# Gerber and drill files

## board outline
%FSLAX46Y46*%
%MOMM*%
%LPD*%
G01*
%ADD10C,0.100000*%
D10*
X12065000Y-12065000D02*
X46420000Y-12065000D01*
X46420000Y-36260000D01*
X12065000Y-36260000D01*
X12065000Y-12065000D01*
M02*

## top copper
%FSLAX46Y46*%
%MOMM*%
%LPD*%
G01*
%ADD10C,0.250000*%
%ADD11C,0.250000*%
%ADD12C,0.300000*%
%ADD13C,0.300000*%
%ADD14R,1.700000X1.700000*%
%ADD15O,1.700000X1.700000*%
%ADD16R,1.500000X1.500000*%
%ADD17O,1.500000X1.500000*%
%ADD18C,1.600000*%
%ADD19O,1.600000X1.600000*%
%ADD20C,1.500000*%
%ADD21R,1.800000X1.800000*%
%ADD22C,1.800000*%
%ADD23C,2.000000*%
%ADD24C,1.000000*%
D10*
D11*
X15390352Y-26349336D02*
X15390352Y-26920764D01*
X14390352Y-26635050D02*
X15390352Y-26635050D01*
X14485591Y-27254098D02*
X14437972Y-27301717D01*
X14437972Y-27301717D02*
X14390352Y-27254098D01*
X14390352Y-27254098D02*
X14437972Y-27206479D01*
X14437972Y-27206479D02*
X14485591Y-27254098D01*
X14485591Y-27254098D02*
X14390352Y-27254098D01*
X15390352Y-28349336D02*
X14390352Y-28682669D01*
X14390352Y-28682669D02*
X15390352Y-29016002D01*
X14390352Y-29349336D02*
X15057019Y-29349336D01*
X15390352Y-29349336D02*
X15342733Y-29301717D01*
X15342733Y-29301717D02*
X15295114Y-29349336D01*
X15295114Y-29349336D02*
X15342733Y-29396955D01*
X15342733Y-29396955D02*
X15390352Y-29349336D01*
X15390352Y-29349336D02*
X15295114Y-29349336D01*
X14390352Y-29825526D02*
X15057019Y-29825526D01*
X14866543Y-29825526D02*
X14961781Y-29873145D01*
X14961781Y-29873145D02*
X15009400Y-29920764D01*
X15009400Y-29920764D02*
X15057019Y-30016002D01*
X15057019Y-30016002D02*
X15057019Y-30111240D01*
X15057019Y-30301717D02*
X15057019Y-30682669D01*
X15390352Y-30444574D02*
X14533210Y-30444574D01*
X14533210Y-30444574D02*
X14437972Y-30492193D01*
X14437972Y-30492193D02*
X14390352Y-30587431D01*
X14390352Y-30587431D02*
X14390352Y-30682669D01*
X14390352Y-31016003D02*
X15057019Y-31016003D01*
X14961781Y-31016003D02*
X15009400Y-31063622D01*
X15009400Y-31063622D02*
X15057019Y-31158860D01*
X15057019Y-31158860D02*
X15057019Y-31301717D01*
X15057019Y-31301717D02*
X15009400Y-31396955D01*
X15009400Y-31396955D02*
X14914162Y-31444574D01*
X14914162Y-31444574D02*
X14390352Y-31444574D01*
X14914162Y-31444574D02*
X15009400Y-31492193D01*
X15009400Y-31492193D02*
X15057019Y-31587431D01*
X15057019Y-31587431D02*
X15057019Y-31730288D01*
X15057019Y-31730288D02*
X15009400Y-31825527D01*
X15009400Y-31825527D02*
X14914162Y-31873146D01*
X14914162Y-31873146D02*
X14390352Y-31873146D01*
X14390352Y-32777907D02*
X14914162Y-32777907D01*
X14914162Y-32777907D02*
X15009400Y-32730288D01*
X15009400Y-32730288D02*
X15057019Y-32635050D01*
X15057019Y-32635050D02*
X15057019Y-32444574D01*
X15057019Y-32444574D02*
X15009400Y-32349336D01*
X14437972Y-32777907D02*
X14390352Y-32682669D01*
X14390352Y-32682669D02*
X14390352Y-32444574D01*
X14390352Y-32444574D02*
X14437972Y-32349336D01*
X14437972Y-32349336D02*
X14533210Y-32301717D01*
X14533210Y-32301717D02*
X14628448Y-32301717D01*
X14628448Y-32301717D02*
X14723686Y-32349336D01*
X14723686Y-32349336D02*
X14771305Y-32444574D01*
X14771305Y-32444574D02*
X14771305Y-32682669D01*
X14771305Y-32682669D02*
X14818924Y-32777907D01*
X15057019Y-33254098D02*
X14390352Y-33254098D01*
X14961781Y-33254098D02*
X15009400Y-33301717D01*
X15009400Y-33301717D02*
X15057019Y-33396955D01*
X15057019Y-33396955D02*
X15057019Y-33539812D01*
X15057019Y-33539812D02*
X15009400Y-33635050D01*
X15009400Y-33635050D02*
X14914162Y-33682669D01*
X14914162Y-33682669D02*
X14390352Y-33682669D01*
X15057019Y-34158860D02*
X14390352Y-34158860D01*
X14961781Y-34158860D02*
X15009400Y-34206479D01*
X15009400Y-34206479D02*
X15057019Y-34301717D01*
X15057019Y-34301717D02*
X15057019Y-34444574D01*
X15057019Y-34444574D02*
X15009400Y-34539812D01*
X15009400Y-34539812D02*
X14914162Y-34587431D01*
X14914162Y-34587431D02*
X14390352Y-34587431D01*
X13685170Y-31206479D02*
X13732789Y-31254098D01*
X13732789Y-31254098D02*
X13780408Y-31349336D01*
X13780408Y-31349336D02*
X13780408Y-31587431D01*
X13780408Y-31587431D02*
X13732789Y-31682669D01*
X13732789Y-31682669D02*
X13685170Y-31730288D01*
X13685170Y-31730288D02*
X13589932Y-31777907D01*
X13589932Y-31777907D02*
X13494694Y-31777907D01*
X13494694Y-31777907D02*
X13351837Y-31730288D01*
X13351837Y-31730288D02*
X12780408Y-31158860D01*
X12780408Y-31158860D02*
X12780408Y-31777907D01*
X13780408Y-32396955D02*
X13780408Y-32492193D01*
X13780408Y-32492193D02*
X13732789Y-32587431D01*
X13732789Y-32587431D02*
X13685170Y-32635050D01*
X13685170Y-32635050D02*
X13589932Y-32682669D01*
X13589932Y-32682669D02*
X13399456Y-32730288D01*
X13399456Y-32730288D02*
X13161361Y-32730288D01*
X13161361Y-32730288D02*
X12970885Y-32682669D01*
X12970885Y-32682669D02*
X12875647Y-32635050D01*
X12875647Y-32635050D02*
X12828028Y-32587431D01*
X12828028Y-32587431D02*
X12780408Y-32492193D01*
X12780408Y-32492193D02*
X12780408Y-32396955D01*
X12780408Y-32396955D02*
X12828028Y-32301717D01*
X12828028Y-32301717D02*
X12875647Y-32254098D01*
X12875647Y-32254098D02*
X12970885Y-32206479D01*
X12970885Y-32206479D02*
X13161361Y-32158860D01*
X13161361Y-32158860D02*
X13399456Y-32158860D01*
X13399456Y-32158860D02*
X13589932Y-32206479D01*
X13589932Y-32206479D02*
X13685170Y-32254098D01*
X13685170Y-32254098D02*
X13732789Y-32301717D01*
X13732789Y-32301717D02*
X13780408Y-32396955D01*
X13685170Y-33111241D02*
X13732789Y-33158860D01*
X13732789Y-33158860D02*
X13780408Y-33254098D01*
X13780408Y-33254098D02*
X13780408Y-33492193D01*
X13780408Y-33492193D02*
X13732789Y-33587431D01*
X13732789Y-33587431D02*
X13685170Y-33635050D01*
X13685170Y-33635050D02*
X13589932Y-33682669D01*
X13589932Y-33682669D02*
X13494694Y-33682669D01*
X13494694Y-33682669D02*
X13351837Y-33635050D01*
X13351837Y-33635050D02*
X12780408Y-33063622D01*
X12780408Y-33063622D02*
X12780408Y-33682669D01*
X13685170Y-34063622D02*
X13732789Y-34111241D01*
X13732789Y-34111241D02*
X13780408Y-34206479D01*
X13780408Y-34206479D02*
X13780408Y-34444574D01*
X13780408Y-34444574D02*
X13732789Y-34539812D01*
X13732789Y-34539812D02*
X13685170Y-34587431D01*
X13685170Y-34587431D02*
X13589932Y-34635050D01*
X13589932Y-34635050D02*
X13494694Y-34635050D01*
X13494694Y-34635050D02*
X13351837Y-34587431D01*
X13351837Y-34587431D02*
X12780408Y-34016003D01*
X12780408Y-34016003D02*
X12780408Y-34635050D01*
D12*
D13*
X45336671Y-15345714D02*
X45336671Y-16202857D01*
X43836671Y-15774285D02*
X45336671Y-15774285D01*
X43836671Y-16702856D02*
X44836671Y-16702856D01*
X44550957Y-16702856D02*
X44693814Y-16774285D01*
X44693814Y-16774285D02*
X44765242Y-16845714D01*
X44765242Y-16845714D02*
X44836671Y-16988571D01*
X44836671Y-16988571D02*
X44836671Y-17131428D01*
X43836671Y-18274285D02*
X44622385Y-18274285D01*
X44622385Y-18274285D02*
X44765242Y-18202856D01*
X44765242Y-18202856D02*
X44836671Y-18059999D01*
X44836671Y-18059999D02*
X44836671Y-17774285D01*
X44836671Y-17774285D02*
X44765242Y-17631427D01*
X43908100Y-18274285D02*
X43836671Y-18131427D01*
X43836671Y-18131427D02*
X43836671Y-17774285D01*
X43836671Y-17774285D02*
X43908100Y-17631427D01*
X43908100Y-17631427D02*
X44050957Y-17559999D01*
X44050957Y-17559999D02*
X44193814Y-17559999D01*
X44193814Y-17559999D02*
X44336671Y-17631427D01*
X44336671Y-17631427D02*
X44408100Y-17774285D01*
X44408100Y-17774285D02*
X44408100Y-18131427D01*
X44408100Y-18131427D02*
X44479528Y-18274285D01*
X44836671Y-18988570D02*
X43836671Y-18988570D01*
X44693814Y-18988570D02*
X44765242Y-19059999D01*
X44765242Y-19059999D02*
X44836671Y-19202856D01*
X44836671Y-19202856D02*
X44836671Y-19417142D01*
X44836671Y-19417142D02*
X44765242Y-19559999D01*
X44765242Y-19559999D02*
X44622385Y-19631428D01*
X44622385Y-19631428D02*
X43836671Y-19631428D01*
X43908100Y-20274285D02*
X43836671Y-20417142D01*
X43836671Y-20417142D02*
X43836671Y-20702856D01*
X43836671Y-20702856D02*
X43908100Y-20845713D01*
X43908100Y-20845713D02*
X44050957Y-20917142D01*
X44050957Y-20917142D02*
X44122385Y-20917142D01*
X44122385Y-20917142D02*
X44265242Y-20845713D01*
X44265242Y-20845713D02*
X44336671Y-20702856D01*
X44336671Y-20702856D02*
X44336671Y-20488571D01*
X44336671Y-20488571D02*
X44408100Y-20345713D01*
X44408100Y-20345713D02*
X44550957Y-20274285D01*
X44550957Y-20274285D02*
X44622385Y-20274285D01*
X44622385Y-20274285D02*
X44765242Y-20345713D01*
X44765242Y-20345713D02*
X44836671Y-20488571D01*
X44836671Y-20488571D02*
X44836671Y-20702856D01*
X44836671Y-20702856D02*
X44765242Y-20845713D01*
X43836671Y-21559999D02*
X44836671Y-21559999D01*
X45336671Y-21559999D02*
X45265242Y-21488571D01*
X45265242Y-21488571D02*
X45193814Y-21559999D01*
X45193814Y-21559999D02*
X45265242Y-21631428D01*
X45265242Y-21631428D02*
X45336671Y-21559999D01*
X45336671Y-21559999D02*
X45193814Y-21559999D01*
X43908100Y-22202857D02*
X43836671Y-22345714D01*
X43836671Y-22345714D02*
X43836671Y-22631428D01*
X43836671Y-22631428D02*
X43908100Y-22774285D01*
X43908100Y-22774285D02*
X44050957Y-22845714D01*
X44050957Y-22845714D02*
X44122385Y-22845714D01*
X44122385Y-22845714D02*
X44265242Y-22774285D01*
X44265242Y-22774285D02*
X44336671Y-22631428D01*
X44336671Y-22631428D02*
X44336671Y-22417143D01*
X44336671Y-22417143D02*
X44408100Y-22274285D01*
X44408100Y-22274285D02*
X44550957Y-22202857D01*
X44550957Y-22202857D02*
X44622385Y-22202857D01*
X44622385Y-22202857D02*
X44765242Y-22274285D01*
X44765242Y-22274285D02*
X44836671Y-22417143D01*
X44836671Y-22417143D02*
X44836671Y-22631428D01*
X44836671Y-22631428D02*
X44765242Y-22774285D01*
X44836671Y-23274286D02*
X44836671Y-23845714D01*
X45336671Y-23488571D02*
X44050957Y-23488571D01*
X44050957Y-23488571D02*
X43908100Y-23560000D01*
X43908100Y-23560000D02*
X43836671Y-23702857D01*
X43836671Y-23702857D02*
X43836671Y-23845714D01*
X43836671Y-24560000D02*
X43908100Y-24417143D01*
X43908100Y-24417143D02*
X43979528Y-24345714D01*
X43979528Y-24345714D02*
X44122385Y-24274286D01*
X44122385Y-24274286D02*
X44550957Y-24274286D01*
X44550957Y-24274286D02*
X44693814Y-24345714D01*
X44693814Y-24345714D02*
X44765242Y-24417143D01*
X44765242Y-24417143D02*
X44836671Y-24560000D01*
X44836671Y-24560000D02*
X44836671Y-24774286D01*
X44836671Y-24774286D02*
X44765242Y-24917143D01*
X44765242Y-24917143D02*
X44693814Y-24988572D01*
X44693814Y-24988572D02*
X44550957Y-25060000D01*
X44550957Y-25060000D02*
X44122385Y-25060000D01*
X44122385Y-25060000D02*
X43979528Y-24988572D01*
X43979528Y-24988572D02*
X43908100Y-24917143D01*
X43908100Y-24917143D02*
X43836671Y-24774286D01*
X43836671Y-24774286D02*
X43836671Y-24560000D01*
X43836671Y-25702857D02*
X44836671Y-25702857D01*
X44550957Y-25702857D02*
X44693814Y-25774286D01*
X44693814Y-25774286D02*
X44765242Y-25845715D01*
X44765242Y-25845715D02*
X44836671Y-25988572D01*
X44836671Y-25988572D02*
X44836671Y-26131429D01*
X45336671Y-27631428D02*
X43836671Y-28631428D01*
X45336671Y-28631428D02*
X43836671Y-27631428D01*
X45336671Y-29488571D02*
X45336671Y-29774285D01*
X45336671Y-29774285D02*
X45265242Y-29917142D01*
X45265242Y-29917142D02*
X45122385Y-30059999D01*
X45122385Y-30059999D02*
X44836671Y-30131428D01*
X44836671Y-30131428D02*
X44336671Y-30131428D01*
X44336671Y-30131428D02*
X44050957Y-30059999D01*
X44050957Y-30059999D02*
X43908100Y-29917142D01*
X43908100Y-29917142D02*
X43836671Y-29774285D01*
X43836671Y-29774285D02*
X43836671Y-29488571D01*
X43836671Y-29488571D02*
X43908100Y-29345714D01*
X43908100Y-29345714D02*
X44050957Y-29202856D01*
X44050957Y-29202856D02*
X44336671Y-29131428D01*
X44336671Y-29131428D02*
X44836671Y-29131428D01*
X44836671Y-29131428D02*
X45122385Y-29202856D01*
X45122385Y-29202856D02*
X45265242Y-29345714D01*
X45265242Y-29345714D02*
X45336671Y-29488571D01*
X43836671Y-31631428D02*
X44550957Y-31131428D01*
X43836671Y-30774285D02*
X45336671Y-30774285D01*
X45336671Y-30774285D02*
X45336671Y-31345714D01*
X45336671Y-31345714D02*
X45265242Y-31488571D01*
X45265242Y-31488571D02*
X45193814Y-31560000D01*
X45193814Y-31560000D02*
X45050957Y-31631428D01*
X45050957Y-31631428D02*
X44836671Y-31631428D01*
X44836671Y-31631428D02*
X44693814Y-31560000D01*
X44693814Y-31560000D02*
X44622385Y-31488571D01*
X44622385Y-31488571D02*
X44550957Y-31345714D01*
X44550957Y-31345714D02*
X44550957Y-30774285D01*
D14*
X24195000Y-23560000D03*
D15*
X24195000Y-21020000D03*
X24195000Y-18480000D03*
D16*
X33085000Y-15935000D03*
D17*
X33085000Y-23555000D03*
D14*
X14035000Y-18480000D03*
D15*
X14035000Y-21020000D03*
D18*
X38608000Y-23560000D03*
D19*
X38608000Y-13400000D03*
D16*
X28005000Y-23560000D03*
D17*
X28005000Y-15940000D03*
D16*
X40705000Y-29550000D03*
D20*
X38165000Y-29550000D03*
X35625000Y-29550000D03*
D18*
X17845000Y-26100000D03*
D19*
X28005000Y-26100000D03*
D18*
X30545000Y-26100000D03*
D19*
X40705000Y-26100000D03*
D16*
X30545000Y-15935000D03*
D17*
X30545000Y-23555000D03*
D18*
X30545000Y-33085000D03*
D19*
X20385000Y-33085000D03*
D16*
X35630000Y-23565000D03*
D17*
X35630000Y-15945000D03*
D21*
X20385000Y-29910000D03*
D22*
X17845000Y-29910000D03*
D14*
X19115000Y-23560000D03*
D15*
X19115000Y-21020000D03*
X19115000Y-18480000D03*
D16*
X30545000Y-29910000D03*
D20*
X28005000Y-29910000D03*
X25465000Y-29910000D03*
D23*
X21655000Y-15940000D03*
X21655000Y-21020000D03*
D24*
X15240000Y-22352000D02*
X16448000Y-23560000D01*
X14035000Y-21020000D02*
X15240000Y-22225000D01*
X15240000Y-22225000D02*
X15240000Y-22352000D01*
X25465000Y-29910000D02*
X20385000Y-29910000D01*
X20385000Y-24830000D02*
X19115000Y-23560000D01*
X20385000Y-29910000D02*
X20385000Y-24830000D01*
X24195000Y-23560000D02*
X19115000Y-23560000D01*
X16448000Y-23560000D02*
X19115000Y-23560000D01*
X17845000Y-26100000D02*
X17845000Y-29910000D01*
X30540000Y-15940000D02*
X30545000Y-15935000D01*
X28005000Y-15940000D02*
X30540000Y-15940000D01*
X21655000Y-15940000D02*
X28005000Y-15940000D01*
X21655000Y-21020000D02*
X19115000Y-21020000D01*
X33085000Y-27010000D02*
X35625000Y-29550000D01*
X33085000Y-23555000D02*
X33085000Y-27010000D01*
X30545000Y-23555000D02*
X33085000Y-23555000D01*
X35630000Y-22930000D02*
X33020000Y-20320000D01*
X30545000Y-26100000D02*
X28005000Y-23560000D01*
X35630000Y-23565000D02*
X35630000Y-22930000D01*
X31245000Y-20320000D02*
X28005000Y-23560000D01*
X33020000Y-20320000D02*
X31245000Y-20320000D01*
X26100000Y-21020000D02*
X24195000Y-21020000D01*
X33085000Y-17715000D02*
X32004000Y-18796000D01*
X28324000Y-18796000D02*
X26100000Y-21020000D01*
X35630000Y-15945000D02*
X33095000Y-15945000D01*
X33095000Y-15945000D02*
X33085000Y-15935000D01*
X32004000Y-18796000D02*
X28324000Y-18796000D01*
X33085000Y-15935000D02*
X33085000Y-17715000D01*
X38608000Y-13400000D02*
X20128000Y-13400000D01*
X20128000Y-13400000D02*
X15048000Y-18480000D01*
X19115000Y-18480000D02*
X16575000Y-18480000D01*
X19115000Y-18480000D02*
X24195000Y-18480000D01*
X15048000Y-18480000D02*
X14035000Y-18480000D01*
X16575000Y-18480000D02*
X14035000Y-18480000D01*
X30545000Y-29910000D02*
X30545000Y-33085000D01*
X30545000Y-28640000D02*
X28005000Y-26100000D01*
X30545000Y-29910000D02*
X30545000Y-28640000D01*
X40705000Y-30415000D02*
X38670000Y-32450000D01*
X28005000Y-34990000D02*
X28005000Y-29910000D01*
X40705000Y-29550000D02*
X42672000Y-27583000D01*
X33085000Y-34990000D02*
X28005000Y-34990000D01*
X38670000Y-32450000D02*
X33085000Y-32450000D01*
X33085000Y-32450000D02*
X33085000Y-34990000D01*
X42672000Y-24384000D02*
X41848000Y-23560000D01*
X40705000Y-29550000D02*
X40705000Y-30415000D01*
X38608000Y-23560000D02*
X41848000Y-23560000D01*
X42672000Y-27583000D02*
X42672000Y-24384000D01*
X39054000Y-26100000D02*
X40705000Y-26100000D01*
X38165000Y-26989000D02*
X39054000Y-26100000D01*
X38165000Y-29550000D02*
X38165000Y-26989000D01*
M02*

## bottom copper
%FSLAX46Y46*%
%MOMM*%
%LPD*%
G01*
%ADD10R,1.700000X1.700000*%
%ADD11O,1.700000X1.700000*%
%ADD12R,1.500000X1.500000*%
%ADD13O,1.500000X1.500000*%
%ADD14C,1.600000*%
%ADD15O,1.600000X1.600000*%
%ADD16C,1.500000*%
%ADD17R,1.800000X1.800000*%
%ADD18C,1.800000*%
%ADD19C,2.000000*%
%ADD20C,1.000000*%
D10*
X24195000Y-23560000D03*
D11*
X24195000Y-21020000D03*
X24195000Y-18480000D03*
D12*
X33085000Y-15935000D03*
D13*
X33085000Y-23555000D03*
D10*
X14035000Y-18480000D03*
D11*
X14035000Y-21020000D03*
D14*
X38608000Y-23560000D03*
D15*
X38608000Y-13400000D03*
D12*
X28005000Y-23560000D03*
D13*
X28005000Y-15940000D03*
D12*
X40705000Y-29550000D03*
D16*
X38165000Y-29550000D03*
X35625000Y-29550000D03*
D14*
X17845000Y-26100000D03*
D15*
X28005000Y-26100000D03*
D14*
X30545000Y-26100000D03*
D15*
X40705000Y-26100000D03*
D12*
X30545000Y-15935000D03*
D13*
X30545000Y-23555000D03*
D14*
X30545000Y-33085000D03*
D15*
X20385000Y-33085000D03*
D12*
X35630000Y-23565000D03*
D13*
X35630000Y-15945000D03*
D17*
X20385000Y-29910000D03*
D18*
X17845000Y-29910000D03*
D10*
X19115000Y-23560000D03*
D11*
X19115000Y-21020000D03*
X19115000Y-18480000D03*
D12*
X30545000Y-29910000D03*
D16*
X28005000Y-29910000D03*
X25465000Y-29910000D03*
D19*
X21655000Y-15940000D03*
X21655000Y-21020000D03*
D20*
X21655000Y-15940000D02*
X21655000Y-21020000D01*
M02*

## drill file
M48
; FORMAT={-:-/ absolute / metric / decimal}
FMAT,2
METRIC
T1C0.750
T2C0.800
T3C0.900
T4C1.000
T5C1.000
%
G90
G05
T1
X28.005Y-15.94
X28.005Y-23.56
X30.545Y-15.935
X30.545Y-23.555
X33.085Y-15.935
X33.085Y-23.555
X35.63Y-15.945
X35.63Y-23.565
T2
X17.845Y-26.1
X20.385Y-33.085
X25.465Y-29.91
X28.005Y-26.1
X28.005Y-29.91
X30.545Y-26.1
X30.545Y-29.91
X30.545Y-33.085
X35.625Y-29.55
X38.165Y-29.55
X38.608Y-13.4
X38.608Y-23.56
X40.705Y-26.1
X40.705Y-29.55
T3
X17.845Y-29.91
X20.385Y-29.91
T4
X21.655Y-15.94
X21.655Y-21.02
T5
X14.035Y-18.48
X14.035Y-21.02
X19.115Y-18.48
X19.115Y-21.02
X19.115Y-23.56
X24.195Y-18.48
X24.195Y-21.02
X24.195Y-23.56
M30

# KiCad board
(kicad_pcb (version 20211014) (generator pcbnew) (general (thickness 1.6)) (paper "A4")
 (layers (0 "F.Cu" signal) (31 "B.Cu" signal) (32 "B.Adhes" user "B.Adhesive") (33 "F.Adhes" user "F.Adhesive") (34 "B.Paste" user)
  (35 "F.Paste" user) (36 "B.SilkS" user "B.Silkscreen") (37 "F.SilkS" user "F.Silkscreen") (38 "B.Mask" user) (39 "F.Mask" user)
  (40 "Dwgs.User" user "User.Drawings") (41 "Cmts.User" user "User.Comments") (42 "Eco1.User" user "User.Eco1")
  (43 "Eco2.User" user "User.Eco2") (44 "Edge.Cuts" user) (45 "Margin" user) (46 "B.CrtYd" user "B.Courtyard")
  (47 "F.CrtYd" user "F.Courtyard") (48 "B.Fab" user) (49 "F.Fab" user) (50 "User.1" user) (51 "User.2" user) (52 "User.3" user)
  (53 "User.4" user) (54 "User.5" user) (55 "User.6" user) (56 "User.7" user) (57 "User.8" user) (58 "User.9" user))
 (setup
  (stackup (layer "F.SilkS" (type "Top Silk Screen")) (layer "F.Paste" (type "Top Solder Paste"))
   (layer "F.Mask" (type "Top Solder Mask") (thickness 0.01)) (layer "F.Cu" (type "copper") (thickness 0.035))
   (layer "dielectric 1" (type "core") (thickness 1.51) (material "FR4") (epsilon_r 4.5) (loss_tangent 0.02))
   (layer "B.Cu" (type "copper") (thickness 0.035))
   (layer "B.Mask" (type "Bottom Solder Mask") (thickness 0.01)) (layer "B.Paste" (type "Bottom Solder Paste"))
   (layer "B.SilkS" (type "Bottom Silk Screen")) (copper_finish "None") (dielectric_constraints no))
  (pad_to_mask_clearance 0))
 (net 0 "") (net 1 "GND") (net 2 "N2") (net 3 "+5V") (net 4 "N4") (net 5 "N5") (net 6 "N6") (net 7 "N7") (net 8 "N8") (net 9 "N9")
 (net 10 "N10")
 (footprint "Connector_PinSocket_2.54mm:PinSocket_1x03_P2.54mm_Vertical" (layer "F.Cu") (at 24.195 23.56 180)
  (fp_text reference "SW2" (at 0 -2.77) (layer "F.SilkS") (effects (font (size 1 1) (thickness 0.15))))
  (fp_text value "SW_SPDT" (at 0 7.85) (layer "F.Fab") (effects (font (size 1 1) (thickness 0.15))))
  (pad "1" thru_hole rect (at 0 0 180) (size 1.7 1.7) (drill 1) (layers *.Cu *.Mask) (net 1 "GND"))
  (pad "2" thru_hole oval (at 0 2.54 180) (size 1.7 1.7) (drill 1) (layers *.Cu *.Mask) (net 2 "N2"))
  (pad "3" thru_hole oval (at 0 5.08 180) (size 1.7 1.7) (drill 1) (layers *.Cu *.Mask) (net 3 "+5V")))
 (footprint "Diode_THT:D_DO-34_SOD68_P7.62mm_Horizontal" (layer "F.Cu") (at 33.085 15.935 -90)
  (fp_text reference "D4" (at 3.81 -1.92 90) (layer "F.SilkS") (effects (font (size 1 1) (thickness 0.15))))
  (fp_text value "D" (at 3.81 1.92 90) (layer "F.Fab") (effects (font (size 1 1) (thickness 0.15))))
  (pad "1" thru_hole rect (at 0 0 270) (size 1.5 1.5) (drill 0.75) (layers *.Cu *.Mask) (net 2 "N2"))
  (pad "2" thru_hole oval (at 7.62 0 270) (size 1.5 1.5) (drill 0.75) (layers *.Cu *.Mask) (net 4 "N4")))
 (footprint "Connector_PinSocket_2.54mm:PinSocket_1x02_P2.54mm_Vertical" (layer "F.Cu") (at 14.035 18.48)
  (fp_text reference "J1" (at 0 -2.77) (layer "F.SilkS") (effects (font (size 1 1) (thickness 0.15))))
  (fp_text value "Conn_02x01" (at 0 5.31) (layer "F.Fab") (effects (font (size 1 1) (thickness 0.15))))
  (pad "1" thru_hole rect (at 0 0) (size 1.7 1.7) (drill 1) (layers *.Cu *.Mask) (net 3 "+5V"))
  (pad "2" thru_hole oval (at 0 2.54) (size 1.7 1.7) (drill 1) (layers *.Cu *.Mask) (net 1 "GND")))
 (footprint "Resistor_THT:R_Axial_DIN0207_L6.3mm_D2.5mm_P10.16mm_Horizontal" (layer "F.Cu") (at 38.608 23.56 90)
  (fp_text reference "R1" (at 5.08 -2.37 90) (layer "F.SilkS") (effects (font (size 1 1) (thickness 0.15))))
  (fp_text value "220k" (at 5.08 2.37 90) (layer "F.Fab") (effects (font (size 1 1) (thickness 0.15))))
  (pad "1" thru_hole circle (at 0 0 90) (size 1.6 1.6) (drill 0.8) (layers *.Cu *.Mask) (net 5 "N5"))
  (pad "2" thru_hole oval (at 10.16 0 90) (size 1.6 1.6) (drill 0.8) (layers *.Cu *.Mask) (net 3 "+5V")))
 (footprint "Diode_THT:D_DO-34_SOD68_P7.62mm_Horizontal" (layer "F.Cu") (at 28.005 23.56 90)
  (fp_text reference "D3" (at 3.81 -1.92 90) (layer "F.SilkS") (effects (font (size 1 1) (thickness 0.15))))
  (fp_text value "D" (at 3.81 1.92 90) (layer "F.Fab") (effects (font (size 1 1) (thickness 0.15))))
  (pad "1" thru_hole rect (at 0 0 90) (size 1.5 1.5) (drill 0.75) (layers *.Cu *.Mask) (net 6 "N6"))
  (pad "2" thru_hole oval (at 7.62 0 90) (size 1.5 1.5) (drill 0.75) (layers *.Cu *.Mask) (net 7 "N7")))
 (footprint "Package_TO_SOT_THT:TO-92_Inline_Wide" (layer "F.Cu") (at 40.705 29.55 180)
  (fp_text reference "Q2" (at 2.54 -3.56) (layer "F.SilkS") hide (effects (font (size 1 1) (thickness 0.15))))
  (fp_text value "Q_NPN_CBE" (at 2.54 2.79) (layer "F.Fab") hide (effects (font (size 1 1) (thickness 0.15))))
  (pad "1" thru_hole rect (at 0 0 180) (size 1.5 1.5) (drill 0.8) (layers *.Cu *.Mask) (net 5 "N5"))
  (pad "2" thru_hole circle (at 2.54 0 180) (size 1.5 1.5) (drill 0.8) (layers *.Cu *.Mask) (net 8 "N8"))
  (pad "3" thru_hole circle (at 5.08 0 180) (size 1.5 1.5) (drill 0.8) (layers *.Cu *.Mask) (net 4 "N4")))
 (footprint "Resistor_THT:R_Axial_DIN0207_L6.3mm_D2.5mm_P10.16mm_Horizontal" (layer "F.Cu") (at 17.845 26.1)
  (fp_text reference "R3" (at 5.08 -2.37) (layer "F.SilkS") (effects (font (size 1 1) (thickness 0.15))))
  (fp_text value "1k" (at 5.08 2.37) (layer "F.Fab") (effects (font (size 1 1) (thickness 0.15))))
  (pad "1" thru_hole circle (at 0 0) (size 1.6 1.6) (drill 0.8) (layers *.Cu *.Mask) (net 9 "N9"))
  (pad "2" thru_hole oval (at 10.16 0) (size 1.6 1.6) (drill 0.8) (layers *.Cu *.Mask) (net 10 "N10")))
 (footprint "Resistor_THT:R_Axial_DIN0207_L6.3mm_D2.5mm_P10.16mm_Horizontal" (layer "F.Cu") (at 30.545 26.1)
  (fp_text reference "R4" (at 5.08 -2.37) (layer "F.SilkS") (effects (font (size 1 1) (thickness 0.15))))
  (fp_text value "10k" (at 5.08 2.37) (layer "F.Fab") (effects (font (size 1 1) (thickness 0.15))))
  (pad "1" thru_hole circle (at 0 0) (size 1.6 1.6) (drill 0.8) (layers *.Cu *.Mask) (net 6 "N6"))
  (pad "2" thru_hole oval (at 10.16 0) (size 1.6 1.6) (drill 0.8) (layers *.Cu *.Mask) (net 8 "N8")))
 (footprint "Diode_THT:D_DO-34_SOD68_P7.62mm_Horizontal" (layer "F.Cu") (at 30.545 15.935 -90)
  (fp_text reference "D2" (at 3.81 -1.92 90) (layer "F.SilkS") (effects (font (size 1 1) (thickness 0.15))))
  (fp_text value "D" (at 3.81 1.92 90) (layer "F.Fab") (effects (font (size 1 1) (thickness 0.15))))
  (pad "1" thru_hole rect (at 0 0 270) (size 1.5 1.5) (drill 0.75) (layers *.Cu *.Mask) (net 7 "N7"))
  (pad "2" thru_hole oval (at 7.62 0 270) (size 1.5 1.5) (drill 0.75) (layers *.Cu *.Mask) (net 4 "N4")))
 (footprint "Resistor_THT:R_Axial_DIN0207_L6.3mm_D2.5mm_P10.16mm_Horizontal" (layer "F.Cu") (at 30.545 33.085 180)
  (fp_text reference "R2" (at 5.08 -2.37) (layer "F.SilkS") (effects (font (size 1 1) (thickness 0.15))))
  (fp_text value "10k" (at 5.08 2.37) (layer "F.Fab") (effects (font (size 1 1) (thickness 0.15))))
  (pad "1" thru_hole circle (at 0 0 180) (size 1.6 1.6) (drill 0.8) (layers *.Cu *.Mask) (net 10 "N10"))
  (pad "2" thru_hole oval (at 10.16 0 180) (size 1.6 1.6) (drill 0.8) (layers *.Cu *.Mask) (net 3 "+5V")))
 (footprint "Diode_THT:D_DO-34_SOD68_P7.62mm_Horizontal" (layer "F.Cu") (at 35.63 23.565 90)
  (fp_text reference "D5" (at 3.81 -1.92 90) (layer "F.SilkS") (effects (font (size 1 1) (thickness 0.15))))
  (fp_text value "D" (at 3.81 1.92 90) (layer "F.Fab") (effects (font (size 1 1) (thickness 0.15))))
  (pad "1" thru_hole rect (at 0 0 90) (size 1.5 1.5) (drill 0.75) (layers *.Cu *.Mask) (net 6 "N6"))
  (pad "2" thru_hole oval (at 7.62 0 90) (size 1.5 1.5) (drill 0.75) (layers *.Cu *.Mask) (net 2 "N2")))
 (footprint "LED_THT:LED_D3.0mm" (layer "F.Cu") (at 20.385 29.91 180)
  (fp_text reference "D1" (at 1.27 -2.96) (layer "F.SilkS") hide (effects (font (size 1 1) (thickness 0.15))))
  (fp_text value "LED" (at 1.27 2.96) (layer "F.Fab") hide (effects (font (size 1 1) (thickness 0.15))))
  (pad "1" thru_hole rect (at 0 0 180) (size 1.8 1.8) (drill 0.9) (layers *.Cu *.Mask) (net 1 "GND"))
  (pad "2" thru_hole circle (at 2.54 0 180) (size 1.8 1.8) (drill 0.9) (layers *.Cu *.Mask) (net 9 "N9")))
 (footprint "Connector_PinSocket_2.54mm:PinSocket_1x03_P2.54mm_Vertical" (layer "F.Cu") (at 19.115 23.56 180)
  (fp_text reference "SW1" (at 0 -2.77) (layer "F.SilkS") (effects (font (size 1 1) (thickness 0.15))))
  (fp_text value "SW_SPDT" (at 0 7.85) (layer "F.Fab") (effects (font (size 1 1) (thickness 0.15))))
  (pad "1" thru_hole rect (at 0 0 180) (size 1.7 1.7) (drill 1) (layers *.Cu *.Mask) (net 1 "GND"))
  (pad "2" thru_hole oval (at 0 2.54 180) (size 1.7 1.7) (drill 1) (layers *.Cu *.Mask) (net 7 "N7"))
  (pad "3" thru_hole oval (at 0 5.08 180) (size 1.7 1.7) (drill 1) (layers *.Cu *.Mask) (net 3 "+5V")))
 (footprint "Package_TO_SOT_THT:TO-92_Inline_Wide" (layer "F.Cu") (at 30.545 29.91 180)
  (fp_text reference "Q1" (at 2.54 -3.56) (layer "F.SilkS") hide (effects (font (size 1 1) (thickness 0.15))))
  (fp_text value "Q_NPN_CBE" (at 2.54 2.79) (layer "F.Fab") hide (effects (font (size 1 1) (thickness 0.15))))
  (pad "1" thru_hole rect (at 0 0 180) (size 1.5 1.5) (drill 0.8) (layers *.Cu *.Mask) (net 10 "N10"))
  (pad "2" thru_hole circle (at 2.54 0 180) (size 1.5 1.5) (drill 0.8) (layers *.Cu *.Mask) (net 5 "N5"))
  (pad "3" thru_hole circle (at 5.08 0 180) (size 1.5 1.5) (drill 0.8) (layers *.Cu *.Mask) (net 1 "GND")))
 (gr_rect (start 12.065 12.065) (end 46.42 36.26) (layer "Edge.Cuts") (width 0.1) (fill none))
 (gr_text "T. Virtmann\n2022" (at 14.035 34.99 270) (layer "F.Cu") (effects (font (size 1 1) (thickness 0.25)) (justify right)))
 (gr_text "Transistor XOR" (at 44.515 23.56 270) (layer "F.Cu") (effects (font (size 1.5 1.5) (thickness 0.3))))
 (segment (start 15.24 22.352) (end 16.448 23.56) (width 1) (layer "F.Cu") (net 1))
 (segment (start 14.035 21.02) (end 15.24 22.225) (width 1) (layer "F.Cu") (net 1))
 (segment (start 15.24 22.225) (end 15.24 22.352) (width 1) (layer "F.Cu") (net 1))
 (segment (start 25.465 29.91) (end 20.385 29.91) (width 1) (layer "F.Cu") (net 1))
 (segment (start 20.385 24.83) (end 19.115 23.56) (width 1) (layer "F.Cu") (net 1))
 (segment (start 20.385 29.91) (end 20.385 24.83) (width 1) (layer "F.Cu") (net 1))
 (segment (start 24.195 23.56) (end 19.115 23.56) (width 1) (layer "F.Cu") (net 1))
 (segment (start 16.448 23.56) (end 19.115 23.56) (width 1) (layer "F.Cu") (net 1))
 (segment (start 17.845 26.1) (end 17.845 29.91) (width 1) (layer "F.Cu") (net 9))
 (segment (start 30.54 15.94) (end 30.545 15.935) (width 1) (layer "F.Cu") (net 7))
 (segment (start 28.005 15.94) (end 30.54 15.94) (width 1) (layer "F.Cu") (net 7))
 (segment (start 21.655 15.94) (end 28.005 15.94) (width 1) (layer "F.Cu") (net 7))
 (segment (start 21.655 21.02) (end 19.115 21.02) (width 1) (layer "F.Cu") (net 7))
 (via (at 21.655 15.94) (size 2) (drill 1) (layers "F.Cu" "B.Cu") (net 7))
 (via (at 21.655 21.02) (size 2) (drill 1) (layers "F.Cu" "B.Cu") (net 7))
 (segment (start 21.655 15.94) (end 21.655 21.02) (width 1) (layer "B.Cu") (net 7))
 (segment (start 33.085 27.01) (end 35.625 29.55) (width 1) (layer "F.Cu") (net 4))
 (segment (start 33.085 23.555) (end 33.085 27.01) (width 1) (layer "F.Cu") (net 4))
 (segment (start 30.545 23.555) (end 33.085 23.555) (width 1) (layer "F.Cu") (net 4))
 (segment (start 35.63 22.93) (end 33.02 20.32) (width 1) (layer "F.Cu") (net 6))
 (segment (start 30.545 26.1) (end 28.005 23.56) (width 1) (layer "F.Cu") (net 6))
 (segment (start 35.63 23.565) (end 35.63 22.93) (width 1) (layer "F.Cu") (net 6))
 (segment (start 31.245 20.32) (end 28.005 23.56) (width 1) (layer "F.Cu") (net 6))
 (segment (start 33.02 20.32) (end 31.245 20.32) (width 1) (layer "F.Cu") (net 6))
 (segment (start 26.1 21.02) (end 24.195 21.02) (width 1) (layer "F.Cu") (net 2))
 (segment (start 33.085 17.715) (end 32.004 18.796) (width 1) (layer "F.Cu") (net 2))
 (segment (start 28.324 18.796) (end 26.1 21.02) (width 1) (layer "F.Cu") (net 2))
 (segment (start 35.63 15.945) (end 33.095 15.945) (width 1) (layer "F.Cu") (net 2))
 (segment (start 33.095 15.945) (end 33.085 15.935) (width 1) (layer "F.Cu") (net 2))
 (segment (start 32.004 18.796) (end 28.324 18.796) (width 1) (layer "F.Cu") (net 2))
 (segment (start 33.085 15.935) (end 33.085 17.715) (width 1) (layer "F.Cu") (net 2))
 (segment (start 38.608 13.4) (end 20.128 13.4) (width 1) (layer "F.Cu") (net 3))
 (segment (start 20.128 13.4) (end 15.048 18.48) (width 1) (layer "F.Cu") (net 3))
 (segment (start 19.115 18.48) (end 16.575 18.48) (width 1) (layer "F.Cu") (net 3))
 (segment (start 19.115 18.48) (end 24.195 18.48) (width 1) (layer "F.Cu") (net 3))
 (segment (start 15.048 18.48) (end 14.035 18.48) (width 1) (layer "F.Cu") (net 3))
 (segment (start 16.575 18.48) (end 14.035 18.48) (width 1) (layer "F.Cu") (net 3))
 (segment (start 30.545 29.91) (end 30.545 33.085) (width 1) (layer "F.Cu") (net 10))
 (segment (start 30.545 28.64) (end 28.005 26.1) (width 1) (layer "F.Cu") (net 10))
 (segment (start 30.545 29.91) (end 30.545 28.64) (width 1) (layer "F.Cu") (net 10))
 (segment (start 40.705 30.415) (end 38.67 32.45) (width 1) (layer "F.Cu") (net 5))
 (segment (start 28.005 34.99) (end 28.005 29.91) (width 1) (layer "F.Cu") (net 5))
 (segment (start 40.705 29.55) (end 42.672 27.583) (width 1) (layer "F.Cu") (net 5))
 (segment (start 33.085 34.99) (end 28.005 34.99) (width 1) (layer "F.Cu") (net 5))
 (segment (start 38.67 32.45) (end 33.085 32.45) (width 1) (layer "F.Cu") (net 5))
 (segment (start 33.085 32.45) (end 33.085 34.99) (width 1) (layer "F.Cu") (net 5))
 (segment (start 42.672 24.384) (end 41.848 23.56) (width 1) (layer "F.Cu") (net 5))
 (segment (start 40.705 29.55) (end 40.705 30.415) (width 1) (layer "F.Cu") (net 5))
 (segment (start 38.608 23.56) (end 41.848 23.56) (width 1) (layer "F.Cu") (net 5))
 (segment (start 42.672 27.583) (end 42.672 24.384) (width 1) (layer "F.Cu") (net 5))
 (segment (start 39.054 26.1) (end 40.705 26.1) (width 1) (layer "F.Cu") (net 8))
 (segment (start 38.165 26.989) (end 39.054 26.1) (width 1) (layer "F.Cu") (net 8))
 (segment (start 38.165 29.55) (end 38.165 26.989) (width 1) (layer "F.Cu") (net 8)))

